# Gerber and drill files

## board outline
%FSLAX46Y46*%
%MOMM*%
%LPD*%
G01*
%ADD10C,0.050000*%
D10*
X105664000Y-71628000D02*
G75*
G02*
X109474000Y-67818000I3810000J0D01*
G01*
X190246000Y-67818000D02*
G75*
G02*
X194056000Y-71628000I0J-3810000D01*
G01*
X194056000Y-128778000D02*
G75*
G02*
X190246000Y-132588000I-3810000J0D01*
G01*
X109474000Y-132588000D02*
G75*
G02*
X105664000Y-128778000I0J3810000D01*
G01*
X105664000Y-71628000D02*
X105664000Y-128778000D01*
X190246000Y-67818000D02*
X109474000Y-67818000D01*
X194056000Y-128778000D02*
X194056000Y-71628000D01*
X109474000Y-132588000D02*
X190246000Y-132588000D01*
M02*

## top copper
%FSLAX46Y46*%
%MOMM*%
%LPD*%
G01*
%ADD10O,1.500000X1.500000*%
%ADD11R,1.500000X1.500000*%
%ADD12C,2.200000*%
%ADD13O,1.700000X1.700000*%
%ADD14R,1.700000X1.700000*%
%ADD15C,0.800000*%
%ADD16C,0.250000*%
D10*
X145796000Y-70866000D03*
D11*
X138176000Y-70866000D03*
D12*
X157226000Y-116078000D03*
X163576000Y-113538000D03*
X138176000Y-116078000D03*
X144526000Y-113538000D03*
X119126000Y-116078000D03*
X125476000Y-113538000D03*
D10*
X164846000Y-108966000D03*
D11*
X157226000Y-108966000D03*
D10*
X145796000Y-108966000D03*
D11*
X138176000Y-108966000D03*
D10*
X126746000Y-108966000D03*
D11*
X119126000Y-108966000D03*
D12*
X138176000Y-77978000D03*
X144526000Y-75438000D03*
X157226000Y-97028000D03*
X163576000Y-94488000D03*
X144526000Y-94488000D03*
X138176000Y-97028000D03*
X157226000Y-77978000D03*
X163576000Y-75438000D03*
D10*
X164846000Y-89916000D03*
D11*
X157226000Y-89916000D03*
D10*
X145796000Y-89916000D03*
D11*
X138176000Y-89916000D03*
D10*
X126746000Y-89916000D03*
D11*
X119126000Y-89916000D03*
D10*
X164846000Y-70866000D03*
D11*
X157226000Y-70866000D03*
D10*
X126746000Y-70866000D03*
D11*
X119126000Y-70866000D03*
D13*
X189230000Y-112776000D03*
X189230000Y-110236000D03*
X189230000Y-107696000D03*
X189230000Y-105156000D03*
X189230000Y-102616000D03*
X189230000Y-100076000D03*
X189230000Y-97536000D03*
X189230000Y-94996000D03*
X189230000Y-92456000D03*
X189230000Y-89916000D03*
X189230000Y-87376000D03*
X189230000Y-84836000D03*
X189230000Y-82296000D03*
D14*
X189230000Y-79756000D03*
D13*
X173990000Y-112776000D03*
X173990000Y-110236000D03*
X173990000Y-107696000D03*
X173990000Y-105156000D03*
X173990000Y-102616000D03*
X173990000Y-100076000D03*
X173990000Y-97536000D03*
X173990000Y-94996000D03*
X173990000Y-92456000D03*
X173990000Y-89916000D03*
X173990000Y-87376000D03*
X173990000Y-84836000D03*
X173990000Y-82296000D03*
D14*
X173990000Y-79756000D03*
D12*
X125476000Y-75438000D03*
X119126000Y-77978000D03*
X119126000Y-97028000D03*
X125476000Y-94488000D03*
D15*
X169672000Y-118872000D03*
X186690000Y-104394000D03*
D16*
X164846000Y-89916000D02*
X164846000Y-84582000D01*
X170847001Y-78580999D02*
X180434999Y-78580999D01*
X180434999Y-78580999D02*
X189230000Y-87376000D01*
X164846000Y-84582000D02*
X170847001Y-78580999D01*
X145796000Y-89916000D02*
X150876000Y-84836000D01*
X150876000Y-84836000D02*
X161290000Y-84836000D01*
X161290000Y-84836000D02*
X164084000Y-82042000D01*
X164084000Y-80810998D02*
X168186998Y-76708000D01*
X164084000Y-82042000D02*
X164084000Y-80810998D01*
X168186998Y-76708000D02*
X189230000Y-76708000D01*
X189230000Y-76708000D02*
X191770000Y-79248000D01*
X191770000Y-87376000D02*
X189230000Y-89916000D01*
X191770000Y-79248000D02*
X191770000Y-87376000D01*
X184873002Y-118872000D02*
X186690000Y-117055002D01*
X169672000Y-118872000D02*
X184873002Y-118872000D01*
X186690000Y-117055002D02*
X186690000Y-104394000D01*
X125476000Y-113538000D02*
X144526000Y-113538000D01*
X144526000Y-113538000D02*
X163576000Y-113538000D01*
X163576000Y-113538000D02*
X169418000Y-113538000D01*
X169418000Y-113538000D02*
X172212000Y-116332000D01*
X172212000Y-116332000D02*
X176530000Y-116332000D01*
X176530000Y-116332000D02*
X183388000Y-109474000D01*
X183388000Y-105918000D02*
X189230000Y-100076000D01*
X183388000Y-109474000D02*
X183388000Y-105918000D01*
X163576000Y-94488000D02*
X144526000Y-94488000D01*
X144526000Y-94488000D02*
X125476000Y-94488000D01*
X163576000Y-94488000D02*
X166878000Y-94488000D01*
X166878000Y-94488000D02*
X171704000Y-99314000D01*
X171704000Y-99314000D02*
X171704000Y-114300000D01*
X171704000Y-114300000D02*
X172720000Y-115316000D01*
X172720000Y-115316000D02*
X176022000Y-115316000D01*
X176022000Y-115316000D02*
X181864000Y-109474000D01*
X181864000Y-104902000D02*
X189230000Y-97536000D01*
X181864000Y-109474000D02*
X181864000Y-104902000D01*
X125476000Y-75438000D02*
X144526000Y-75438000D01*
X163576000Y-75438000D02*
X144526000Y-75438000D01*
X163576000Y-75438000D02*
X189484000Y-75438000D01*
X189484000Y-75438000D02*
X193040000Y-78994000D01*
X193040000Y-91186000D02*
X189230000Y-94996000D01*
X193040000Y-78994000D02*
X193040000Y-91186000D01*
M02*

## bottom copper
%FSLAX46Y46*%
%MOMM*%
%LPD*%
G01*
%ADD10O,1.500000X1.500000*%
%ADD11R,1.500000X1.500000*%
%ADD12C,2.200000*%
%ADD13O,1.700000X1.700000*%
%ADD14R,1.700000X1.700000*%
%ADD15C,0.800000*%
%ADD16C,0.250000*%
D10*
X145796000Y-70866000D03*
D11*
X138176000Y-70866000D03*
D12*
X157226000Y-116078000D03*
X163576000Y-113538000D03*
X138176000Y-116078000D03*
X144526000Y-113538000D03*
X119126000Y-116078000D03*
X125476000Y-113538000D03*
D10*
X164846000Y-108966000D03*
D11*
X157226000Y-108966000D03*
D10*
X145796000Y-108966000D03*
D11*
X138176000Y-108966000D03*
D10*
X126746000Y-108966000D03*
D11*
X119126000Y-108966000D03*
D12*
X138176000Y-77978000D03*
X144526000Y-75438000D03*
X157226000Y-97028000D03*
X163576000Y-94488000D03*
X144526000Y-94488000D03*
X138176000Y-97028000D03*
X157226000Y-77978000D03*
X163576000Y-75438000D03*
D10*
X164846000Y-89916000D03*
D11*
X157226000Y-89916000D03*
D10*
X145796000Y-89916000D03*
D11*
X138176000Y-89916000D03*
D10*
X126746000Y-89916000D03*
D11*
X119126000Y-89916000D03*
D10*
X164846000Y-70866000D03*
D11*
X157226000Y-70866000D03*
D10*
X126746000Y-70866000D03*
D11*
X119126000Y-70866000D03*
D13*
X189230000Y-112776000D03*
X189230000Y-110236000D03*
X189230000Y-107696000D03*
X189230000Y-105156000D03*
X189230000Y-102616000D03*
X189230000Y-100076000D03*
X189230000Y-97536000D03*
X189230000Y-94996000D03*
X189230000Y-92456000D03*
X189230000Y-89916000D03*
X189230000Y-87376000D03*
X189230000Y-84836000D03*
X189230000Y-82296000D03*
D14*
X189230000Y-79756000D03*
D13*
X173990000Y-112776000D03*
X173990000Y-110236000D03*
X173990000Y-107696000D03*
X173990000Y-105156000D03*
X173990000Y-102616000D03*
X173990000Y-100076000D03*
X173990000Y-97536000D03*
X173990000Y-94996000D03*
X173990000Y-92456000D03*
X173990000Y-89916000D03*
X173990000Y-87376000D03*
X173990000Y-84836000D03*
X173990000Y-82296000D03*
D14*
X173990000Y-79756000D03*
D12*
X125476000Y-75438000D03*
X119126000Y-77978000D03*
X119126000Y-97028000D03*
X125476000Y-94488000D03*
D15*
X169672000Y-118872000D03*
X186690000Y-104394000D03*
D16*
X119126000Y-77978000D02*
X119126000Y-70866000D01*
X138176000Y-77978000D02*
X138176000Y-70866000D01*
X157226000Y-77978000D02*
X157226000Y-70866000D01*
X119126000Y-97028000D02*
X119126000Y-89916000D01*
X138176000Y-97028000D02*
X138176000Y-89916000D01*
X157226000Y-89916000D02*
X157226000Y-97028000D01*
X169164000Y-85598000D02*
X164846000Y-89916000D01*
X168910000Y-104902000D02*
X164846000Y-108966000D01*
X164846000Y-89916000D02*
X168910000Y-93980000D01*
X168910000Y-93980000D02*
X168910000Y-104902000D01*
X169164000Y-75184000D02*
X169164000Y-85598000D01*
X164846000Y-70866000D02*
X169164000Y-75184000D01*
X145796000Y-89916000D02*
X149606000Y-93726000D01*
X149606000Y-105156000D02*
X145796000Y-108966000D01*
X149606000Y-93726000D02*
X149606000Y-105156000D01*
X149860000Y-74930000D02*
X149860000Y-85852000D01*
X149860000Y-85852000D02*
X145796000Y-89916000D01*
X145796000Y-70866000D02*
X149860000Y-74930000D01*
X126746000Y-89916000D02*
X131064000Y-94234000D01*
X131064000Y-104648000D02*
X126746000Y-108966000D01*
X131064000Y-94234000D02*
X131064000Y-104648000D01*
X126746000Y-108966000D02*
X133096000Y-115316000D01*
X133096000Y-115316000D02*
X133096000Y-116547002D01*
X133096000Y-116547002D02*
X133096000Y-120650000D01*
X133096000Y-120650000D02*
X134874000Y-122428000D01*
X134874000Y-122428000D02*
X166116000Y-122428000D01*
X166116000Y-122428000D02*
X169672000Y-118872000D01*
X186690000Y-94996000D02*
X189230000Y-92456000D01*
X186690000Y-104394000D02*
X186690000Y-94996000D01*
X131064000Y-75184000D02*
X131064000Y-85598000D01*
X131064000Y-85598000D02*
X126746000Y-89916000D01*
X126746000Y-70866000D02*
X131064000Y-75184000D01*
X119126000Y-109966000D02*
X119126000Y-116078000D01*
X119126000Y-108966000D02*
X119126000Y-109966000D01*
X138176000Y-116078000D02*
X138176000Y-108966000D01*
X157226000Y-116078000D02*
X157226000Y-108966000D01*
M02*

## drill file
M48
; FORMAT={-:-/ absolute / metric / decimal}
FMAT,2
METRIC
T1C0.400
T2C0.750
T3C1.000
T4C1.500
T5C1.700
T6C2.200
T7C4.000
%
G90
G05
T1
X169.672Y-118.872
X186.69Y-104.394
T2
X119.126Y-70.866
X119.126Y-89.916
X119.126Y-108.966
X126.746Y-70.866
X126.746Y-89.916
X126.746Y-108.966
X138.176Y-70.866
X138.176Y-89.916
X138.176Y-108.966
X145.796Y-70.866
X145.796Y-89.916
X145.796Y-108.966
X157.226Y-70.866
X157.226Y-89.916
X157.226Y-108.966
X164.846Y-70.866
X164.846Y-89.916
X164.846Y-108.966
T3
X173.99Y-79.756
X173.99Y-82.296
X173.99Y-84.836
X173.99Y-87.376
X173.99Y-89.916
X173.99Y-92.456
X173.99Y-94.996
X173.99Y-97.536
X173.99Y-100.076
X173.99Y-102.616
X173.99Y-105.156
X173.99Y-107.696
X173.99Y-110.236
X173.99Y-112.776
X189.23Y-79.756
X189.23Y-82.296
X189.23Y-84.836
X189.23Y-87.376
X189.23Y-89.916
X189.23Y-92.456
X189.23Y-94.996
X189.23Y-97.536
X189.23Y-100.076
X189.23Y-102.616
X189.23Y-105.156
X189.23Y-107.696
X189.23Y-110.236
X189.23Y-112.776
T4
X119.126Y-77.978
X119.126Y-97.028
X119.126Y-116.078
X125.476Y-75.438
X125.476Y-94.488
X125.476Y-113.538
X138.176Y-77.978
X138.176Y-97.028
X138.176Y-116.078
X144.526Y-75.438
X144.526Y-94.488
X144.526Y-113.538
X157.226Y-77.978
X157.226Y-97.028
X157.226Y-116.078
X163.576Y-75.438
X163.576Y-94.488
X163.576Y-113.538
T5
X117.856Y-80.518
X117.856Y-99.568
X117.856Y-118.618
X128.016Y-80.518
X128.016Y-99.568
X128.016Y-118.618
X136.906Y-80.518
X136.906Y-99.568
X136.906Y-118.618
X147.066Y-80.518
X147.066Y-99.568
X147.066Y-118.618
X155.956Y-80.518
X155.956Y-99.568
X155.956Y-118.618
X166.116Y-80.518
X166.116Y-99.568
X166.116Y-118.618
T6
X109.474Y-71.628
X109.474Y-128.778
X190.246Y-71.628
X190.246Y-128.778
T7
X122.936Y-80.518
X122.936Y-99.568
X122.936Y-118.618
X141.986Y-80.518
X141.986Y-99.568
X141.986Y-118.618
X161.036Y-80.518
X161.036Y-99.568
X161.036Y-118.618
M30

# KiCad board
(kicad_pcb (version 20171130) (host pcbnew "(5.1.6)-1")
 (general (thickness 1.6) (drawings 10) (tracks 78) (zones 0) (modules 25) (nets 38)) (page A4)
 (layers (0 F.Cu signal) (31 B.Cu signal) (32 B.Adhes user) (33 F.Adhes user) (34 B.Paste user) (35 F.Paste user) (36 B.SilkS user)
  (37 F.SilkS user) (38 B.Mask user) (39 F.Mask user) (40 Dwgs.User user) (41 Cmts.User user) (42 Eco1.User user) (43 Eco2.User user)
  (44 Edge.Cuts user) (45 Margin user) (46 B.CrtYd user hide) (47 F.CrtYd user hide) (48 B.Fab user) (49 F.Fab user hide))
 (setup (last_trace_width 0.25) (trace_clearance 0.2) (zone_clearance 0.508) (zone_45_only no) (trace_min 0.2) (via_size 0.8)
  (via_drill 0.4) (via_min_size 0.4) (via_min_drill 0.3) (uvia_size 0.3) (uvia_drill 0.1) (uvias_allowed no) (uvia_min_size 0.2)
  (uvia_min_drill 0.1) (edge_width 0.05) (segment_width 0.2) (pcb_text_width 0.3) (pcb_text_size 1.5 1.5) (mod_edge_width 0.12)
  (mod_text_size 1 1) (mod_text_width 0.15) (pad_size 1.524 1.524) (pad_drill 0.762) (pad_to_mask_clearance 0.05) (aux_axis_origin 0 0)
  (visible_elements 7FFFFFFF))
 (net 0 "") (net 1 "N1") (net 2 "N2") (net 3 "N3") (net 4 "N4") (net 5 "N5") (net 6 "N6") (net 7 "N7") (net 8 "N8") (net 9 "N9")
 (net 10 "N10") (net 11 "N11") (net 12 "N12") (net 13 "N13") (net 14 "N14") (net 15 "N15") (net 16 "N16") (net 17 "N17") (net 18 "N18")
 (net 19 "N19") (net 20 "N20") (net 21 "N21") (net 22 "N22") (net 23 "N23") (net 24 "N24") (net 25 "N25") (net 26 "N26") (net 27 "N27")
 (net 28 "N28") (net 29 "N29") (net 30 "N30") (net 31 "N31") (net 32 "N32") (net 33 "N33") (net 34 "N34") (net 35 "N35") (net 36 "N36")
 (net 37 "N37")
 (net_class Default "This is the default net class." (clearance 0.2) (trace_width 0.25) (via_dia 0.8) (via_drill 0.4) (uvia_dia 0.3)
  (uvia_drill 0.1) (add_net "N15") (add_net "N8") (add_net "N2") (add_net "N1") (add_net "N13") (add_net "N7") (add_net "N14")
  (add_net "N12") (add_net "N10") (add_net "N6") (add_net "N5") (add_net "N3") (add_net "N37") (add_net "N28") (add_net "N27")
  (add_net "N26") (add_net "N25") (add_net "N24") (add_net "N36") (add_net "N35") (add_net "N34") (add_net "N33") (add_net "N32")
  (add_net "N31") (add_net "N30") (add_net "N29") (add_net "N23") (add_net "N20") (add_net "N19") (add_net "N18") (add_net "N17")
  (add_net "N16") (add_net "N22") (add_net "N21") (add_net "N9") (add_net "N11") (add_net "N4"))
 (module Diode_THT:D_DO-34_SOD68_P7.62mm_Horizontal (layer F.Cu) (at 138.176 70.866)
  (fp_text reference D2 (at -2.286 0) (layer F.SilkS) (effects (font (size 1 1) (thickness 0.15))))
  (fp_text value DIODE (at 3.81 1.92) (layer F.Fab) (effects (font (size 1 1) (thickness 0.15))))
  (pad 2 thru_hole oval (at 7.62 0) (size 1.5 1.5) (drill 0.75) (layers *.Cu *.Mask) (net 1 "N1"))
  (pad 1 thru_hole rect (at 0 0) (size 1.5 1.5) (drill 0.75) (layers *.Cu *.Mask) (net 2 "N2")))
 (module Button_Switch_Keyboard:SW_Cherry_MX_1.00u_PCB (layer F.Cu) (at 163.576 113.538)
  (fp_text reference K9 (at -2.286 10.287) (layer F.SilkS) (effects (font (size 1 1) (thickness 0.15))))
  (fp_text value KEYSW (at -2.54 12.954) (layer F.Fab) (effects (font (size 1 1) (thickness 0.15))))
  (pad "" np_thru_hole circle (at 2.54 5.08) (size 1.7 1.7) (drill 1.7) (layers *.Cu *.Mask))
  (pad "" np_thru_hole circle (at -7.62 5.08) (size 1.7 1.7) (drill 1.7) (layers *.Cu *.Mask))
  (pad "" np_thru_hole circle (at -2.54 5.08) (size 4 4) (drill 4) (layers *.Cu *.Mask))
  (pad 2 thru_hole circle (at -6.35 2.54) (size 2.2 2.2) (drill 1.5) (layers *.Cu *.Mask) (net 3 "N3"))
  (pad 1 thru_hole circle (at 0 0) (size 2.2 2.2) (drill 1.5) (layers *.Cu *.Mask) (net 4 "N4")))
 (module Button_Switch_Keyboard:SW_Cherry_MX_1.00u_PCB (layer F.Cu) (at 144.526 113.538)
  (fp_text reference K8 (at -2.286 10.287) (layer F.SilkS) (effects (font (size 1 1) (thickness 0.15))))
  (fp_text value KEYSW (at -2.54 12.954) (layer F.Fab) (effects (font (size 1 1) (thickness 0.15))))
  (pad "" np_thru_hole circle (at 2.54 5.08) (size 1.7 1.7) (drill 1.7) (layers *.Cu *.Mask))
  (pad "" np_thru_hole circle (at -7.62 5.08) (size 1.7 1.7) (drill 1.7) (layers *.Cu *.Mask))
  (pad "" np_thru_hole circle (at -2.54 5.08) (size 4 4) (drill 4) (layers *.Cu *.Mask))
  (pad 2 thru_hole circle (at -6.35 2.54) (size 2.2 2.2) (drill 1.5) (layers *.Cu *.Mask) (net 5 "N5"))
  (pad 1 thru_hole circle (at 0 0) (size 2.2 2.2) (drill 1.5) (layers *.Cu *.Mask) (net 4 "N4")))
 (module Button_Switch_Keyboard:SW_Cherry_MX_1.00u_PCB (layer F.Cu) (at 125.476 113.538)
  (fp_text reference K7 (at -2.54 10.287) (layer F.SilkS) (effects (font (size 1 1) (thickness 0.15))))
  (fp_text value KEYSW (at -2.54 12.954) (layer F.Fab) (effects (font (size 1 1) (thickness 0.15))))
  (pad "" np_thru_hole circle (at 2.54 5.08) (size 1.7 1.7) (drill 1.7) (layers *.Cu *.Mask))
  (pad "" np_thru_hole circle (at -7.62 5.08) (size 1.7 1.7) (drill 1.7) (layers *.Cu *.Mask))
  (pad "" np_thru_hole circle (at -2.54 5.08) (size 4 4) (drill 4) (layers *.Cu *.Mask))
  (pad 2 thru_hole circle (at -6.35 2.54) (size 2.2 2.2) (drill 1.5) (layers *.Cu *.Mask) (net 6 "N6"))
  (pad 1 thru_hole circle (at 0 0) (size 2.2 2.2) (drill 1.5) (layers *.Cu *.Mask) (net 4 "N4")))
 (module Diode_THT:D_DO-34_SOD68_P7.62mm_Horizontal (layer F.Cu) (at 157.226 108.966)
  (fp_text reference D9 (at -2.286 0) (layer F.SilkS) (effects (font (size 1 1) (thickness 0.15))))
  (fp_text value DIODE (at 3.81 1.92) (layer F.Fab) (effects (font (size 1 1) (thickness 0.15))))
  (pad 2 thru_hole oval (at 7.62 0) (size 1.5 1.5) (drill 0.75) (layers *.Cu *.Mask) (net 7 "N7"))
  (pad 1 thru_hole rect (at 0 0) (size 1.5 1.5) (drill 0.75) (layers *.Cu *.Mask) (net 3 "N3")))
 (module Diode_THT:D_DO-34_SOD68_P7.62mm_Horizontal (layer F.Cu) (at 138.176 108.966)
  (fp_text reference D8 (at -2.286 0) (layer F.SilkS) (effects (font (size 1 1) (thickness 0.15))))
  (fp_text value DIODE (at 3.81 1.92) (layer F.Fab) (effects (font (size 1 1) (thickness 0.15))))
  (pad 2 thru_hole oval (at 7.62 0) (size 1.5 1.5) (drill 0.75) (layers *.Cu *.Mask) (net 1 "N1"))
  (pad 1 thru_hole rect (at 0 0) (size 1.5 1.5) (drill 0.75) (layers *.Cu *.Mask) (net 5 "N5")))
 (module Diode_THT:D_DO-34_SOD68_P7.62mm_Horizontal (layer F.Cu) (at 119.126 108.966)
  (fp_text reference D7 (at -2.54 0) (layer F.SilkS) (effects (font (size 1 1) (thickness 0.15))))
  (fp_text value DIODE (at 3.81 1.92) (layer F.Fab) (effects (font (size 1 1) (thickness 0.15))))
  (pad 2 thru_hole oval (at 7.62 0) (size 1.5 1.5) (drill 0.75) (layers *.Cu *.Mask) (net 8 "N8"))
  (pad 1 thru_hole rect (at 0 0) (size 1.5 1.5) (drill 0.75) (layers *.Cu *.Mask) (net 6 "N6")))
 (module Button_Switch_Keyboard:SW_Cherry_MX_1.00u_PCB (layer F.Cu) (at 144.526 75.438)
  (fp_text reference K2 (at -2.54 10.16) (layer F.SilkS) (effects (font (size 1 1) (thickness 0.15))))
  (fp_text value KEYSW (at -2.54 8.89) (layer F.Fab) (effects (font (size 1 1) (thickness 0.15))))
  (pad "" np_thru_hole circle (at 2.54 5.08) (size 1.7 1.7) (drill 1.7) (layers *.Cu *.Mask))
  (pad "" np_thru_hole circle (at -7.62 5.08) (size 1.7 1.7) (drill 1.7) (layers *.Cu *.Mask))
  (pad "" np_thru_hole circle (at -2.54 5.08) (size 4 4) (drill 4) (layers *.Cu *.Mask))
  (pad 2 thru_hole circle (at -6.35 2.54) (size 2.2 2.2) (drill 1.5) (layers *.Cu *.Mask) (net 2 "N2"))
  (pad 1 thru_hole circle (at 0 0) (size 2.2 2.2) (drill 1.5) (layers *.Cu *.Mask) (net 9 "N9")))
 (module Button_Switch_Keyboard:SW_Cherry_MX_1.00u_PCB (layer F.Cu) (at 163.576 94.488)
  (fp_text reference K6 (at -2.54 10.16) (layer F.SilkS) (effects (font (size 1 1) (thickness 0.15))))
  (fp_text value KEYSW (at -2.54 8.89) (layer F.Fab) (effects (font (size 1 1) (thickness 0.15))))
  (pad "" np_thru_hole circle (at 2.54 5.08) (size 1.7 1.7) (drill 1.7) (layers *.Cu *.Mask))
  (pad "" np_thru_hole circle (at -7.62 5.08) (size 1.7 1.7) (drill 1.7) (layers *.Cu *.Mask))
  (pad "" np_thru_hole circle (at -2.54 5.08) (size 4 4) (drill 4) (layers *.Cu *.Mask))
  (pad 2 thru_hole circle (at -6.35 2.54) (size 2.2 2.2) (drill 1.5) (layers *.Cu *.Mask) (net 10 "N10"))
  (pad 1 thru_hole circle (at 0 0) (size 2.2 2.2) (drill 1.5) (layers *.Cu *.Mask) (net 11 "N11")))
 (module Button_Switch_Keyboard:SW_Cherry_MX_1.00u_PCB (layer F.Cu) (at 144.526 94.488)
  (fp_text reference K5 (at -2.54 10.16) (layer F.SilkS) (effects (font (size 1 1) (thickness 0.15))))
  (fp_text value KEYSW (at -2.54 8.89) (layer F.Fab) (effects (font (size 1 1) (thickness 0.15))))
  (pad 1 thru_hole circle (at 0 0) (size 2.2 2.2) (drill 1.5) (layers *.Cu *.Mask) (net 11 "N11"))
  (pad 2 thru_hole circle (at -6.35 2.54) (size 2.2 2.2) (drill 1.5) (layers *.Cu *.Mask) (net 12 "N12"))
  (pad "" np_thru_hole circle (at -2.54 5.08) (size 4 4) (drill 4) (layers *.Cu *.Mask))
  (pad "" np_thru_hole circle (at -7.62 5.08) (size 1.7 1.7) (drill 1.7) (layers *.Cu *.Mask))
  (pad "" np_thru_hole circle (at 2.54 5.08) (size 1.7 1.7) (drill 1.7) (layers *.Cu *.Mask)))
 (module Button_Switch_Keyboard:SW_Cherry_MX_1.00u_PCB (layer F.Cu) (at 163.576 75.438)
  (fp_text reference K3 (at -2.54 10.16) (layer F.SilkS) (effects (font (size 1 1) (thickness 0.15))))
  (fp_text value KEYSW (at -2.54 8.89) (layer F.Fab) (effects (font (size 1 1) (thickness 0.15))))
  (pad "" np_thru_hole circle (at 2.54 5.08) (size 1.7 1.7) (drill 1.7) (layers *.Cu *.Mask))
  (pad "" np_thru_hole circle (at -7.62 5.08) (size 1.7 1.7) (drill 1.7) (layers *.Cu *.Mask))
  (pad "" np_thru_hole circle (at -2.54 5.08) (size 4 4) (drill 4) (layers *.Cu *.Mask))
  (pad 2 thru_hole circle (at -6.35 2.54) (size 2.2 2.2) (drill 1.5) (layers *.Cu *.Mask) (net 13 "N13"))
  (pad 1 thru_hole circle (at 0 0) (size 2.2 2.2) (drill 1.5) (layers *.Cu *.Mask) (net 9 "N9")))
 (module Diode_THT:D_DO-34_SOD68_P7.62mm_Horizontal (layer F.Cu) (at 157.226 89.916)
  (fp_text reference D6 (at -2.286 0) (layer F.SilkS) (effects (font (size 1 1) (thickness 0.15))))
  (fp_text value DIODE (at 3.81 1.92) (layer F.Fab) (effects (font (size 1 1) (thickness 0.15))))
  (pad 2 thru_hole oval (at 7.62 0) (size 1.5 1.5) (drill 0.75) (layers *.Cu *.Mask) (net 7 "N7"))
  (pad 1 thru_hole rect (at 0 0) (size 1.5 1.5) (drill 0.75) (layers *.Cu *.Mask) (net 10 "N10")))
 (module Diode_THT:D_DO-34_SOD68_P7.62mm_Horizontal (layer F.Cu) (at 138.176 89.916)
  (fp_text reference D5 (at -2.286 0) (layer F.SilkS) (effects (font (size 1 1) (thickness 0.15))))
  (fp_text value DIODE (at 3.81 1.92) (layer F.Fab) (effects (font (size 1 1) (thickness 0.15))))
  (pad 2 thru_hole oval (at 7.62 0) (size 1.5 1.5) (drill 0.75) (layers *.Cu *.Mask) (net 1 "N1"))
  (pad 1 thru_hole rect (at 0 0) (size 1.5 1.5) (drill 0.75) (layers *.Cu *.Mask) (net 12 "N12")))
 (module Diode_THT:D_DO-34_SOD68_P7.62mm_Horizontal (layer F.Cu) (at 119.126 89.916)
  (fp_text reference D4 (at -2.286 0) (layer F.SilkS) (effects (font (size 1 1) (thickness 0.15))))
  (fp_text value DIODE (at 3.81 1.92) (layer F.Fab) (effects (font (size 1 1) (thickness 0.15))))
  (pad 2 thru_hole oval (at 7.62 0) (size 1.5 1.5) (drill 0.75) (layers *.Cu *.Mask) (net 8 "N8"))
  (pad 1 thru_hole rect (at 0 0) (size 1.5 1.5) (drill 0.75) (layers *.Cu *.Mask) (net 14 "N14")))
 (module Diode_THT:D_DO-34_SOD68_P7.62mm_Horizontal (layer F.Cu) (at 157.226 70.866)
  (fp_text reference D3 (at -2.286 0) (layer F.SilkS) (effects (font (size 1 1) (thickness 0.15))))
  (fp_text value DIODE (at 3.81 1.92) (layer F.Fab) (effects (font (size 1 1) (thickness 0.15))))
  (pad 2 thru_hole oval (at 7.62 0) (size 1.5 1.5) (drill 0.75) (layers *.Cu *.Mask) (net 7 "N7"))
  (pad 1 thru_hole rect (at 0 0) (size 1.5 1.5) (drill 0.75) (layers *.Cu *.Mask) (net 13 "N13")))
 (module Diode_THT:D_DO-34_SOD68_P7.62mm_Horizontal (layer F.Cu) (at 119.126 70.866)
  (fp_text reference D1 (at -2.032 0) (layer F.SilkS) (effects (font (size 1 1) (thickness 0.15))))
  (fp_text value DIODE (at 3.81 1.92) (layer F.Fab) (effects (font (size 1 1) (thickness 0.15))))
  (pad 2 thru_hole oval (at 7.62 0) (size 1.5 1.5) (drill 0.75) (layers *.Cu *.Mask) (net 8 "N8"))
  (pad 1 thru_hole rect (at 0 0) (size 1.5 1.5) (drill 0.75) (layers *.Cu *.Mask) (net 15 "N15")))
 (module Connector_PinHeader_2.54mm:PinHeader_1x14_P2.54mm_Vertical (layer F.Cu) (at 189.23 79.756)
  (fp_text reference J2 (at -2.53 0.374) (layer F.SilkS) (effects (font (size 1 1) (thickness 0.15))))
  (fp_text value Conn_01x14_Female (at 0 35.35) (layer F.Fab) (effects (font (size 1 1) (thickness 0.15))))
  (pad 14 thru_hole oval (at 0 33.02) (size 1.7 1.7) (drill 1) (layers *.Cu *.Mask) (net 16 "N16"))
  (pad 13 thru_hole oval (at 0 30.48) (size 1.7 1.7) (drill 1) (layers *.Cu *.Mask) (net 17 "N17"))
  (pad 12 thru_hole oval (at 0 27.94) (size 1.7 1.7) (drill 1) (layers *.Cu *.Mask) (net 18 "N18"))
  (pad 11 thru_hole oval (at 0 25.4) (size 1.7 1.7) (drill 1) (layers *.Cu *.Mask) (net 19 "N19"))
  (pad 10 thru_hole oval (at 0 22.86) (size 1.7 1.7) (drill 1) (layers *.Cu *.Mask) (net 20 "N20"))
  (pad 9 thru_hole oval (at 0 20.32) (size 1.7 1.7) (drill 1) (layers *.Cu *.Mask) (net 4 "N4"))
  (pad 8 thru_hole oval (at 0 17.78) (size 1.7 1.7) (drill 1) (layers *.Cu *.Mask) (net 11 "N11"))
  (pad 7 thru_hole oval (at 0 15.24) (size 1.7 1.7) (drill 1) (layers *.Cu *.Mask) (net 9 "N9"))
  (pad 6 thru_hole oval (at 0 12.7) (size 1.7 1.7) (drill 1) (layers *.Cu *.Mask) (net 8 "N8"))
  (pad 5 thru_hole oval (at 0 10.16) (size 1.7 1.7) (drill 1) (layers *.Cu *.Mask) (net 1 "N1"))
  (pad 4 thru_hole oval (at 0 7.62) (size 1.7 1.7) (drill 1) (layers *.Cu *.Mask) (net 7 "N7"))
  (pad 3 thru_hole oval (at 0 5.08) (size 1.7 1.7) (drill 1) (layers *.Cu *.Mask) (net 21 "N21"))
  (pad 2 thru_hole oval (at 0 2.54) (size 1.7 1.7) (drill 1) (layers *.Cu *.Mask) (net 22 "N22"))
  (pad 1 thru_hole rect (at 0 0) (size 1.7 1.7) (drill 1) (layers *.Cu *.Mask) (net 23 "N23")))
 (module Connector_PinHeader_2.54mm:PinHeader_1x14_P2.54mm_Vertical (layer F.Cu) (at 173.99 79.756)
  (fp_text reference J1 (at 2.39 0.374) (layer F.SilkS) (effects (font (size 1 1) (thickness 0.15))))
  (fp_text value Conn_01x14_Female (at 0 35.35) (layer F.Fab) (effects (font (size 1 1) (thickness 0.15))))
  (pad 14 thru_hole oval (at 0 33.02) (size 1.7 1.7) (drill 1) (layers *.Cu *.Mask) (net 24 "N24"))
  (pad 13 thru_hole oval (at 0 30.48) (size 1.7 1.7) (drill 1) (layers *.Cu *.Mask) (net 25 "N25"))
  (pad 12 thru_hole oval (at 0 27.94) (size 1.7 1.7) (drill 1) (layers *.Cu *.Mask) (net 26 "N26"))
  (pad 11 thru_hole oval (at 0 25.4) (size 1.7 1.7) (drill 1) (layers *.Cu *.Mask) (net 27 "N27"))
  (pad 10 thru_hole oval (at 0 22.86) (size 1.7 1.7) (drill 1) (layers *.Cu *.Mask) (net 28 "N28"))
  (pad 9 thru_hole oval (at 0 20.32) (size 1.7 1.7) (drill 1) (layers *.Cu *.Mask) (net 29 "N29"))
  (pad 8 thru_hole oval (at 0 17.78) (size 1.7 1.7) (drill 1) (layers *.Cu *.Mask) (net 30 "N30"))
  (pad 7 thru_hole oval (at 0 15.24) (size 1.7 1.7) (drill 1) (layers *.Cu *.Mask) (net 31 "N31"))
  (pad 6 thru_hole oval (at 0 12.7) (size 1.7 1.7) (drill 1) (layers *.Cu *.Mask) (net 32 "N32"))
  (pad 5 thru_hole oval (at 0 10.16) (size 1.7 1.7) (drill 1) (layers *.Cu *.Mask) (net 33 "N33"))
  (pad 4 thru_hole oval (at 0 7.62) (size 1.7 1.7) (drill 1) (layers *.Cu *.Mask) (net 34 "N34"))
  (pad 3 thru_hole oval (at 0 5.08) (size 1.7 1.7) (drill 1) (layers *.Cu *.Mask) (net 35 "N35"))
  (pad 2 thru_hole oval (at 0 2.54) (size 1.7 1.7) (drill 1) (layers *.Cu *.Mask) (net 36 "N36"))
  (pad 1 thru_hole rect (at 0 0) (size 1.7 1.7) (drill 1) (layers *.Cu *.Mask) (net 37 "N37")))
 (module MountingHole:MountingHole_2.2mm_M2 (layer F.Cu) (at 109.474 71.628)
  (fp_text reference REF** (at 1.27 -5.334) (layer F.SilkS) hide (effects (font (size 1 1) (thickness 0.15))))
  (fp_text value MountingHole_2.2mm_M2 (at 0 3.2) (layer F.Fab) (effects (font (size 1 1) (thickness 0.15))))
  (pad 1 np_thru_hole circle (at 0 0) (size 2.2 2.2) (drill 2.2) (layers *.Cu *.Mask)))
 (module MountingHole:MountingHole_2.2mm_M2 (layer F.Cu) (at 109.474 128.778)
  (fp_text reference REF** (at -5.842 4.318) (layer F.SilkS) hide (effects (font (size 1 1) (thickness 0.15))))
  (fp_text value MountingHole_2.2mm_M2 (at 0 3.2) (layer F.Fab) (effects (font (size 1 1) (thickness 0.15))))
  (pad 1 np_thru_hole circle (at 0 0) (size 2.2 2.2) (drill 2.2) (layers *.Cu *.Mask)))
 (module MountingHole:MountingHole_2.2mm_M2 (layer F.Cu) (at 190.246 128.778)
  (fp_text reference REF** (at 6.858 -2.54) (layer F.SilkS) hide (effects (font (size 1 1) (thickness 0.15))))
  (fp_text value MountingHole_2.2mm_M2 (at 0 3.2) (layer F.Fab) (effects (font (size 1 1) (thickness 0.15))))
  (pad 1 np_thru_hole circle (at 0 0) (size 2.2 2.2) (drill 2.2) (layers *.Cu *.Mask)))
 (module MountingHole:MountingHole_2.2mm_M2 (layer F.Cu) (at 190.246 71.628)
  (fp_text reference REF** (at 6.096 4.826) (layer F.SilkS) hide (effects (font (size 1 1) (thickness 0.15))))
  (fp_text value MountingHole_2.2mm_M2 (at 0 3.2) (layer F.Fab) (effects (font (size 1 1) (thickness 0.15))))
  (pad 1 np_thru_hole circle (at 0 0) (size 2.2 2.2) (drill 2.2) (layers *.Cu *.Mask)))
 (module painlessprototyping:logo (layer B.Cu) (at 181.67 85.14 270)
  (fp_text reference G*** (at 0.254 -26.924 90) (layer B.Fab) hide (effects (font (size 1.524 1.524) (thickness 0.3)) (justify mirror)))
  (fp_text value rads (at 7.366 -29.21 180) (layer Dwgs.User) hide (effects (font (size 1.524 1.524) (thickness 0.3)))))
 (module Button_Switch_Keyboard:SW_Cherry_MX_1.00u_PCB (layer F.Cu) (at 125.476 75.438)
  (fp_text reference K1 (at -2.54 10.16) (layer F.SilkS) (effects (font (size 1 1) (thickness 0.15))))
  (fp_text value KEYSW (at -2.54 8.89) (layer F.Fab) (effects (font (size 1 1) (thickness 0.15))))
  (pad 1 thru_hole circle (at 0 0) (size 2.2 2.2) (drill 1.5) (layers *.Cu *.Mask) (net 9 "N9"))
  (pad 2 thru_hole circle (at -6.35 2.54) (size 2.2 2.2) (drill 1.5) (layers *.Cu *.Mask) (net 15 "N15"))
  (pad "" np_thru_hole circle (at -2.54 5.08) (size 4 4) (drill 4) (layers *.Cu *.Mask))
  (pad "" np_thru_hole circle (at -7.62 5.08) (size 1.7 1.7) (drill 1.7) (layers *.Cu *.Mask))
  (pad "" np_thru_hole circle (at 2.54 5.08) (size 1.7 1.7) (drill 1.7) (layers *.Cu *.Mask)))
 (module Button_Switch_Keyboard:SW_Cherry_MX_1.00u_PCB (layer F.Cu) (at 125.476 94.488)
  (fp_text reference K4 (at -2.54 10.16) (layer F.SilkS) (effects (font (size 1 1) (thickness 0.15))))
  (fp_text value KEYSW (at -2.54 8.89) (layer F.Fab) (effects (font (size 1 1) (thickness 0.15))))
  (pad "" np_thru_hole circle (at 2.54 5.08) (size 1.7 1.7) (drill 1.7) (layers *.Cu *.Mask))
  (pad "" np_thru_hole circle (at -7.62 5.08) (size 1.7 1.7) (drill 1.7) (layers *.Cu *.Mask))
  (pad "" np_thru_hole circle (at -2.54 5.08) (size 4 4) (drill 4) (layers *.Cu *.Mask))
  (pad 2 thru_hole circle (at -6.35 2.54) (size 2.2 2.2) (drill 1.5) (layers *.Cu *.Mask) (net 14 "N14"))
  (pad 1 thru_hole circle (at 0 0) (size 2.2 2.2) (drill 1.5) (layers *.Cu *.Mask) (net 11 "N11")))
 (gr_arc (start 109.474 71.628) (end 109.474 67.818) (angle -90) (layer Edge.Cuts) (width 0.05))
 (gr_arc (start 190.246 71.628) (end 194.056 71.628) (angle -90) (layer Edge.Cuts) (width 0.05))
 (gr_arc (start 190.246 128.778) (end 190.246 132.588) (angle -90) (layer Edge.Cuts) (width 0.05))
 (gr_arc (start 109.474 128.778) (end 105.664 128.778) (angle -90) (layer Edge.Cuts) (width 0.05))
 (gr_line (start 105.664 71.628) (end 105.664 128.778) (layer Edge.Cuts) (width 0.05))
 (gr_line (start 190.246 67.818) (end 109.474 67.818) (layer Edge.Cuts) (width 0.05))
 (gr_line (start 194.056 128.778) (end 194.056 71.628) (layer Edge.Cuts) (width 0.05))
 (gr_line (start 109.474 132.588) (end 190.246 132.588) (layer Edge.Cuts) (width 0.05))
 (segment (start 119.126 77.978) (end 119.126 70.866) (width 0.25) (layer B.Cu) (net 15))
 (segment (start 138.176 77.978) (end 138.176 70.866) (width 0.25) (layer B.Cu) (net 2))
 (segment (start 157.226 77.978) (end 157.226 70.866) (width 0.25) (layer B.Cu) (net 13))
 (segment (start 119.126 97.028) (end 119.126 89.916) (width 0.25) (layer B.Cu) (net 14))
 (segment (start 138.176 97.028) (end 138.176 89.916) (width 0.25) (layer B.Cu) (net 12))
 (segment (start 157.226 89.916) (end 157.226 97.028) (width 0.25) (layer B.Cu) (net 10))
 (segment (start 169.164 85.598) (end 164.846 89.916) (width 0.25) (layer B.Cu) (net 7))
 (segment (start 168.91 104.902) (end 164.846 108.966) (width 0.25) (layer B.Cu) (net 7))
 (segment (start 164.846 89.916) (end 168.91 93.98) (width 0.25) (layer B.Cu) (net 7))
 (segment (start 168.91 93.98) (end 168.91 104.902) (width 0.25) (layer B.Cu) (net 7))
 (segment (start 164.846 89.916) (end 164.846 84.582) (width 0.25) (layer F.Cu) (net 7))
 (segment (start 170.847001 78.580999) (end 180.434999 78.580999) (width 0.25) (layer F.Cu) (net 7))
 (segment (start 180.434999 78.580999) (end 189.23 87.376) (width 0.25) (layer F.Cu) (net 7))
 (segment (start 164.846 84.582) (end 170.847001 78.580999) (width 0.25) (layer F.Cu) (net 7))
 (segment (start 169.164 75.184) (end 169.164 85.598) (width 0.25) (layer B.Cu) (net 7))
 (segment (start 164.846 70.866) (end 169.164 75.184) (width 0.25) (layer B.Cu) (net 7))
 (segment (start 145.796 89.916) (end 149.606 93.726) (width 0.25) (layer B.Cu) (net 1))
 (segment (start 149.606 105.156) (end 145.796 108.966) (width 0.25) (layer B.Cu) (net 1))
 (segment (start 149.606 93.726) (end 149.606 105.156) (width 0.25) (layer B.Cu) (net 1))
 (segment (start 145.796 89.916) (end 150.876 84.836) (width 0.25) (layer F.Cu) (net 1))
 (segment (start 150.876 84.836) (end 161.29 84.836) (width 0.25) (layer F.Cu) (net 1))
 (segment (start 161.29 84.836) (end 164.084 82.042) (width 0.25) (layer F.Cu) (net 1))
 (segment (start 164.084 80.810998) (end 168.186998 76.708) (width 0.25) (layer F.Cu) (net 1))
 (segment (start 164.084 82.042) (end 164.084 80.810998) (width 0.25) (layer F.Cu) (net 1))
 (segment (start 168.186998 76.708) (end 189.23 76.708) (width 0.25) (layer F.Cu) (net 1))
 (segment (start 189.23 76.708) (end 191.77 79.248) (width 0.25) (layer F.Cu) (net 1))
 (segment (start 191.77 87.376) (end 189.23 89.916) (width 0.25) (layer F.Cu) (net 1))
 (segment (start 191.77 79.248) (end 191.77 87.376) (width 0.25) (layer F.Cu) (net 1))
 (segment (start 149.86 74.93) (end 149.86 85.852) (width 0.25) (layer B.Cu) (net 1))
 (segment (start 149.86 85.852) (end 145.796 89.916) (width 0.25) (layer B.Cu) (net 1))
 (segment (start 145.796 70.866) (end 149.86 74.93) (width 0.25) (layer B.Cu) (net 1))
 (segment (start 126.746 89.916) (end 131.064 94.234) (width 0.25) (layer B.Cu) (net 8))
 (segment (start 131.064 104.648) (end 126.746 108.966) (width 0.25) (layer B.Cu) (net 8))
 (segment (start 131.064 94.234) (end 131.064 104.648) (width 0.25) (layer B.Cu) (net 8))
 (segment (start 126.746 108.966) (end 133.096 115.316) (width 0.25) (layer B.Cu) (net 8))
 (segment (start 133.096 115.316) (end 133.096 116.547002) (width 0.25) (layer B.Cu) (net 8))
 (segment (start 133.096 116.547002) (end 133.096 120.65) (width 0.25) (layer B.Cu) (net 8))
 (segment (start 133.096 120.65) (end 134.874 122.428) (width 0.25) (layer B.Cu) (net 8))
 (segment (start 134.874 122.428) (end 166.116 122.428) (width 0.25) (layer B.Cu) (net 8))
 (via (at 169.672 118.872) (size 0.8) (drill 0.4) (layers F.Cu B.Cu) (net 8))
 (segment (start 166.116 122.428) (end 169.672 118.872) (width 0.25) (layer B.Cu) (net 8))
 (segment (start 184.873002 118.872) (end 186.69 117.055002) (width 0.25) (layer F.Cu) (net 8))
 (segment (start 169.672 118.872) (end 184.873002 118.872) (width 0.25) (layer F.Cu) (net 8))
 (via (at 186.69 104.394) (size 0.8) (drill 0.4) (layers F.Cu B.Cu) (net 8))
 (segment (start 186.69 117.055002) (end 186.69 104.394) (width 0.25) (layer F.Cu) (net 8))
 (segment (start 186.69 94.996) (end 189.23 92.456) (width 0.25) (layer B.Cu) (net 8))
 (segment (start 186.69 104.394) (end 186.69 94.996) (width 0.25) (layer B.Cu) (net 8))
 (segment (start 131.064 75.184) (end 131.064 85.598) (width 0.25) (layer B.Cu) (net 8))
 (segment (start 131.064 85.598) (end 126.746 89.916) (width 0.25) (layer B.Cu) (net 8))
 (segment (start 126.746 70.866) (end 131.064 75.184) (width 0.25) (layer B.Cu) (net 8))
 (segment (start 125.476 113.538) (end 144.526 113.538) (width 0.25) (layer F.Cu) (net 4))
 (segment (start 144.526 113.538) (end 163.576 113.538) (width 0.25) (layer F.Cu) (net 4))
 (segment (start 163.576 113.538) (end 169.418 113.538) (width 0.25) (layer F.Cu) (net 4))
 (segment (start 169.418 113.538) (end 172.212 116.332) (width 0.25) (layer F.Cu) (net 4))
 (segment (start 172.212 116.332) (end 176.53 116.332) (width 0.25) (layer F.Cu) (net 4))
 (segment (start 176.53 116.332) (end 183.388 109.474) (width 0.25) (layer F.Cu) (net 4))
 (segment (start 183.388 105.918) (end 189.23 100.076) (width 0.25) (layer F.Cu) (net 4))
 (segment (start 183.388 109.474) (end 183.388 105.918) (width 0.25) (layer F.Cu) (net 4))
 (segment (start 163.576 94.488) (end 144.526 94.488) (width 0.25) (layer F.Cu) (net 11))
 (segment (start 144.526 94.488) (end 125.476 94.488) (width 0.25) (layer F.Cu) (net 11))
 (segment (start 163.576 94.488) (end 166.878 94.488) (width 0.25) (layer F.Cu) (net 11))
 (segment (start 166.878 94.488) (end 171.704 99.314) (width 0.25) (layer F.Cu) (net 11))
 (segment (start 171.704 99.314) (end 171.704 114.3) (width 0.25) (layer F.Cu) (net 11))
 (segment (start 171.704 114.3) (end 172.72 115.316) (width 0.25) (layer F.Cu) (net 11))
 (segment (start 172.72 115.316) (end 176.022 115.316) (width 0.25) (layer F.Cu) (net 11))
 (segment (start 176.022 115.316) (end 181.864 109.474) (width 0.25) (layer F.Cu) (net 11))
 (segment (start 181.864 104.902) (end 189.23 97.536) (width 0.25) (layer F.Cu) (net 11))
 (segment (start 181.864 109.474) (end 181.864 104.902) (width 0.25) (layer F.Cu) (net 11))
 (segment (start 125.476 75.438) (end 144.526 75.438) (width 0.25) (layer F.Cu) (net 9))
 (segment (start 163.576 75.438) (end 144.526 75.438) (width 0.25) (layer F.Cu) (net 9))
 (segment (start 163.576 75.438) (end 189.484 75.438) (width 0.25) (layer F.Cu) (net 9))
 (segment (start 189.484 75.438) (end 193.04 78.994) (width 0.25) (layer F.Cu) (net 9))
 (segment (start 193.04 91.186) (end 189.23 94.996) (width 0.25) (layer F.Cu) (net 9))
 (segment (start 193.04 78.994) (end 193.04 91.186) (width 0.25) (layer F.Cu) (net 9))
 (segment (start 119.126 109.966) (end 119.126 116.078) (width 0.25) (layer B.Cu) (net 6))
 (segment (start 119.126 108.966) (end 119.126 109.966) (width 0.25) (layer B.Cu) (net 6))
 (segment (start 138.176 116.078) (end 138.176 108.966) (width 0.25) (layer B.Cu) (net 5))
 (segment (start 157.226 116.078) (end 157.226 108.966) (width 0.25) (layer B.Cu) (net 3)))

